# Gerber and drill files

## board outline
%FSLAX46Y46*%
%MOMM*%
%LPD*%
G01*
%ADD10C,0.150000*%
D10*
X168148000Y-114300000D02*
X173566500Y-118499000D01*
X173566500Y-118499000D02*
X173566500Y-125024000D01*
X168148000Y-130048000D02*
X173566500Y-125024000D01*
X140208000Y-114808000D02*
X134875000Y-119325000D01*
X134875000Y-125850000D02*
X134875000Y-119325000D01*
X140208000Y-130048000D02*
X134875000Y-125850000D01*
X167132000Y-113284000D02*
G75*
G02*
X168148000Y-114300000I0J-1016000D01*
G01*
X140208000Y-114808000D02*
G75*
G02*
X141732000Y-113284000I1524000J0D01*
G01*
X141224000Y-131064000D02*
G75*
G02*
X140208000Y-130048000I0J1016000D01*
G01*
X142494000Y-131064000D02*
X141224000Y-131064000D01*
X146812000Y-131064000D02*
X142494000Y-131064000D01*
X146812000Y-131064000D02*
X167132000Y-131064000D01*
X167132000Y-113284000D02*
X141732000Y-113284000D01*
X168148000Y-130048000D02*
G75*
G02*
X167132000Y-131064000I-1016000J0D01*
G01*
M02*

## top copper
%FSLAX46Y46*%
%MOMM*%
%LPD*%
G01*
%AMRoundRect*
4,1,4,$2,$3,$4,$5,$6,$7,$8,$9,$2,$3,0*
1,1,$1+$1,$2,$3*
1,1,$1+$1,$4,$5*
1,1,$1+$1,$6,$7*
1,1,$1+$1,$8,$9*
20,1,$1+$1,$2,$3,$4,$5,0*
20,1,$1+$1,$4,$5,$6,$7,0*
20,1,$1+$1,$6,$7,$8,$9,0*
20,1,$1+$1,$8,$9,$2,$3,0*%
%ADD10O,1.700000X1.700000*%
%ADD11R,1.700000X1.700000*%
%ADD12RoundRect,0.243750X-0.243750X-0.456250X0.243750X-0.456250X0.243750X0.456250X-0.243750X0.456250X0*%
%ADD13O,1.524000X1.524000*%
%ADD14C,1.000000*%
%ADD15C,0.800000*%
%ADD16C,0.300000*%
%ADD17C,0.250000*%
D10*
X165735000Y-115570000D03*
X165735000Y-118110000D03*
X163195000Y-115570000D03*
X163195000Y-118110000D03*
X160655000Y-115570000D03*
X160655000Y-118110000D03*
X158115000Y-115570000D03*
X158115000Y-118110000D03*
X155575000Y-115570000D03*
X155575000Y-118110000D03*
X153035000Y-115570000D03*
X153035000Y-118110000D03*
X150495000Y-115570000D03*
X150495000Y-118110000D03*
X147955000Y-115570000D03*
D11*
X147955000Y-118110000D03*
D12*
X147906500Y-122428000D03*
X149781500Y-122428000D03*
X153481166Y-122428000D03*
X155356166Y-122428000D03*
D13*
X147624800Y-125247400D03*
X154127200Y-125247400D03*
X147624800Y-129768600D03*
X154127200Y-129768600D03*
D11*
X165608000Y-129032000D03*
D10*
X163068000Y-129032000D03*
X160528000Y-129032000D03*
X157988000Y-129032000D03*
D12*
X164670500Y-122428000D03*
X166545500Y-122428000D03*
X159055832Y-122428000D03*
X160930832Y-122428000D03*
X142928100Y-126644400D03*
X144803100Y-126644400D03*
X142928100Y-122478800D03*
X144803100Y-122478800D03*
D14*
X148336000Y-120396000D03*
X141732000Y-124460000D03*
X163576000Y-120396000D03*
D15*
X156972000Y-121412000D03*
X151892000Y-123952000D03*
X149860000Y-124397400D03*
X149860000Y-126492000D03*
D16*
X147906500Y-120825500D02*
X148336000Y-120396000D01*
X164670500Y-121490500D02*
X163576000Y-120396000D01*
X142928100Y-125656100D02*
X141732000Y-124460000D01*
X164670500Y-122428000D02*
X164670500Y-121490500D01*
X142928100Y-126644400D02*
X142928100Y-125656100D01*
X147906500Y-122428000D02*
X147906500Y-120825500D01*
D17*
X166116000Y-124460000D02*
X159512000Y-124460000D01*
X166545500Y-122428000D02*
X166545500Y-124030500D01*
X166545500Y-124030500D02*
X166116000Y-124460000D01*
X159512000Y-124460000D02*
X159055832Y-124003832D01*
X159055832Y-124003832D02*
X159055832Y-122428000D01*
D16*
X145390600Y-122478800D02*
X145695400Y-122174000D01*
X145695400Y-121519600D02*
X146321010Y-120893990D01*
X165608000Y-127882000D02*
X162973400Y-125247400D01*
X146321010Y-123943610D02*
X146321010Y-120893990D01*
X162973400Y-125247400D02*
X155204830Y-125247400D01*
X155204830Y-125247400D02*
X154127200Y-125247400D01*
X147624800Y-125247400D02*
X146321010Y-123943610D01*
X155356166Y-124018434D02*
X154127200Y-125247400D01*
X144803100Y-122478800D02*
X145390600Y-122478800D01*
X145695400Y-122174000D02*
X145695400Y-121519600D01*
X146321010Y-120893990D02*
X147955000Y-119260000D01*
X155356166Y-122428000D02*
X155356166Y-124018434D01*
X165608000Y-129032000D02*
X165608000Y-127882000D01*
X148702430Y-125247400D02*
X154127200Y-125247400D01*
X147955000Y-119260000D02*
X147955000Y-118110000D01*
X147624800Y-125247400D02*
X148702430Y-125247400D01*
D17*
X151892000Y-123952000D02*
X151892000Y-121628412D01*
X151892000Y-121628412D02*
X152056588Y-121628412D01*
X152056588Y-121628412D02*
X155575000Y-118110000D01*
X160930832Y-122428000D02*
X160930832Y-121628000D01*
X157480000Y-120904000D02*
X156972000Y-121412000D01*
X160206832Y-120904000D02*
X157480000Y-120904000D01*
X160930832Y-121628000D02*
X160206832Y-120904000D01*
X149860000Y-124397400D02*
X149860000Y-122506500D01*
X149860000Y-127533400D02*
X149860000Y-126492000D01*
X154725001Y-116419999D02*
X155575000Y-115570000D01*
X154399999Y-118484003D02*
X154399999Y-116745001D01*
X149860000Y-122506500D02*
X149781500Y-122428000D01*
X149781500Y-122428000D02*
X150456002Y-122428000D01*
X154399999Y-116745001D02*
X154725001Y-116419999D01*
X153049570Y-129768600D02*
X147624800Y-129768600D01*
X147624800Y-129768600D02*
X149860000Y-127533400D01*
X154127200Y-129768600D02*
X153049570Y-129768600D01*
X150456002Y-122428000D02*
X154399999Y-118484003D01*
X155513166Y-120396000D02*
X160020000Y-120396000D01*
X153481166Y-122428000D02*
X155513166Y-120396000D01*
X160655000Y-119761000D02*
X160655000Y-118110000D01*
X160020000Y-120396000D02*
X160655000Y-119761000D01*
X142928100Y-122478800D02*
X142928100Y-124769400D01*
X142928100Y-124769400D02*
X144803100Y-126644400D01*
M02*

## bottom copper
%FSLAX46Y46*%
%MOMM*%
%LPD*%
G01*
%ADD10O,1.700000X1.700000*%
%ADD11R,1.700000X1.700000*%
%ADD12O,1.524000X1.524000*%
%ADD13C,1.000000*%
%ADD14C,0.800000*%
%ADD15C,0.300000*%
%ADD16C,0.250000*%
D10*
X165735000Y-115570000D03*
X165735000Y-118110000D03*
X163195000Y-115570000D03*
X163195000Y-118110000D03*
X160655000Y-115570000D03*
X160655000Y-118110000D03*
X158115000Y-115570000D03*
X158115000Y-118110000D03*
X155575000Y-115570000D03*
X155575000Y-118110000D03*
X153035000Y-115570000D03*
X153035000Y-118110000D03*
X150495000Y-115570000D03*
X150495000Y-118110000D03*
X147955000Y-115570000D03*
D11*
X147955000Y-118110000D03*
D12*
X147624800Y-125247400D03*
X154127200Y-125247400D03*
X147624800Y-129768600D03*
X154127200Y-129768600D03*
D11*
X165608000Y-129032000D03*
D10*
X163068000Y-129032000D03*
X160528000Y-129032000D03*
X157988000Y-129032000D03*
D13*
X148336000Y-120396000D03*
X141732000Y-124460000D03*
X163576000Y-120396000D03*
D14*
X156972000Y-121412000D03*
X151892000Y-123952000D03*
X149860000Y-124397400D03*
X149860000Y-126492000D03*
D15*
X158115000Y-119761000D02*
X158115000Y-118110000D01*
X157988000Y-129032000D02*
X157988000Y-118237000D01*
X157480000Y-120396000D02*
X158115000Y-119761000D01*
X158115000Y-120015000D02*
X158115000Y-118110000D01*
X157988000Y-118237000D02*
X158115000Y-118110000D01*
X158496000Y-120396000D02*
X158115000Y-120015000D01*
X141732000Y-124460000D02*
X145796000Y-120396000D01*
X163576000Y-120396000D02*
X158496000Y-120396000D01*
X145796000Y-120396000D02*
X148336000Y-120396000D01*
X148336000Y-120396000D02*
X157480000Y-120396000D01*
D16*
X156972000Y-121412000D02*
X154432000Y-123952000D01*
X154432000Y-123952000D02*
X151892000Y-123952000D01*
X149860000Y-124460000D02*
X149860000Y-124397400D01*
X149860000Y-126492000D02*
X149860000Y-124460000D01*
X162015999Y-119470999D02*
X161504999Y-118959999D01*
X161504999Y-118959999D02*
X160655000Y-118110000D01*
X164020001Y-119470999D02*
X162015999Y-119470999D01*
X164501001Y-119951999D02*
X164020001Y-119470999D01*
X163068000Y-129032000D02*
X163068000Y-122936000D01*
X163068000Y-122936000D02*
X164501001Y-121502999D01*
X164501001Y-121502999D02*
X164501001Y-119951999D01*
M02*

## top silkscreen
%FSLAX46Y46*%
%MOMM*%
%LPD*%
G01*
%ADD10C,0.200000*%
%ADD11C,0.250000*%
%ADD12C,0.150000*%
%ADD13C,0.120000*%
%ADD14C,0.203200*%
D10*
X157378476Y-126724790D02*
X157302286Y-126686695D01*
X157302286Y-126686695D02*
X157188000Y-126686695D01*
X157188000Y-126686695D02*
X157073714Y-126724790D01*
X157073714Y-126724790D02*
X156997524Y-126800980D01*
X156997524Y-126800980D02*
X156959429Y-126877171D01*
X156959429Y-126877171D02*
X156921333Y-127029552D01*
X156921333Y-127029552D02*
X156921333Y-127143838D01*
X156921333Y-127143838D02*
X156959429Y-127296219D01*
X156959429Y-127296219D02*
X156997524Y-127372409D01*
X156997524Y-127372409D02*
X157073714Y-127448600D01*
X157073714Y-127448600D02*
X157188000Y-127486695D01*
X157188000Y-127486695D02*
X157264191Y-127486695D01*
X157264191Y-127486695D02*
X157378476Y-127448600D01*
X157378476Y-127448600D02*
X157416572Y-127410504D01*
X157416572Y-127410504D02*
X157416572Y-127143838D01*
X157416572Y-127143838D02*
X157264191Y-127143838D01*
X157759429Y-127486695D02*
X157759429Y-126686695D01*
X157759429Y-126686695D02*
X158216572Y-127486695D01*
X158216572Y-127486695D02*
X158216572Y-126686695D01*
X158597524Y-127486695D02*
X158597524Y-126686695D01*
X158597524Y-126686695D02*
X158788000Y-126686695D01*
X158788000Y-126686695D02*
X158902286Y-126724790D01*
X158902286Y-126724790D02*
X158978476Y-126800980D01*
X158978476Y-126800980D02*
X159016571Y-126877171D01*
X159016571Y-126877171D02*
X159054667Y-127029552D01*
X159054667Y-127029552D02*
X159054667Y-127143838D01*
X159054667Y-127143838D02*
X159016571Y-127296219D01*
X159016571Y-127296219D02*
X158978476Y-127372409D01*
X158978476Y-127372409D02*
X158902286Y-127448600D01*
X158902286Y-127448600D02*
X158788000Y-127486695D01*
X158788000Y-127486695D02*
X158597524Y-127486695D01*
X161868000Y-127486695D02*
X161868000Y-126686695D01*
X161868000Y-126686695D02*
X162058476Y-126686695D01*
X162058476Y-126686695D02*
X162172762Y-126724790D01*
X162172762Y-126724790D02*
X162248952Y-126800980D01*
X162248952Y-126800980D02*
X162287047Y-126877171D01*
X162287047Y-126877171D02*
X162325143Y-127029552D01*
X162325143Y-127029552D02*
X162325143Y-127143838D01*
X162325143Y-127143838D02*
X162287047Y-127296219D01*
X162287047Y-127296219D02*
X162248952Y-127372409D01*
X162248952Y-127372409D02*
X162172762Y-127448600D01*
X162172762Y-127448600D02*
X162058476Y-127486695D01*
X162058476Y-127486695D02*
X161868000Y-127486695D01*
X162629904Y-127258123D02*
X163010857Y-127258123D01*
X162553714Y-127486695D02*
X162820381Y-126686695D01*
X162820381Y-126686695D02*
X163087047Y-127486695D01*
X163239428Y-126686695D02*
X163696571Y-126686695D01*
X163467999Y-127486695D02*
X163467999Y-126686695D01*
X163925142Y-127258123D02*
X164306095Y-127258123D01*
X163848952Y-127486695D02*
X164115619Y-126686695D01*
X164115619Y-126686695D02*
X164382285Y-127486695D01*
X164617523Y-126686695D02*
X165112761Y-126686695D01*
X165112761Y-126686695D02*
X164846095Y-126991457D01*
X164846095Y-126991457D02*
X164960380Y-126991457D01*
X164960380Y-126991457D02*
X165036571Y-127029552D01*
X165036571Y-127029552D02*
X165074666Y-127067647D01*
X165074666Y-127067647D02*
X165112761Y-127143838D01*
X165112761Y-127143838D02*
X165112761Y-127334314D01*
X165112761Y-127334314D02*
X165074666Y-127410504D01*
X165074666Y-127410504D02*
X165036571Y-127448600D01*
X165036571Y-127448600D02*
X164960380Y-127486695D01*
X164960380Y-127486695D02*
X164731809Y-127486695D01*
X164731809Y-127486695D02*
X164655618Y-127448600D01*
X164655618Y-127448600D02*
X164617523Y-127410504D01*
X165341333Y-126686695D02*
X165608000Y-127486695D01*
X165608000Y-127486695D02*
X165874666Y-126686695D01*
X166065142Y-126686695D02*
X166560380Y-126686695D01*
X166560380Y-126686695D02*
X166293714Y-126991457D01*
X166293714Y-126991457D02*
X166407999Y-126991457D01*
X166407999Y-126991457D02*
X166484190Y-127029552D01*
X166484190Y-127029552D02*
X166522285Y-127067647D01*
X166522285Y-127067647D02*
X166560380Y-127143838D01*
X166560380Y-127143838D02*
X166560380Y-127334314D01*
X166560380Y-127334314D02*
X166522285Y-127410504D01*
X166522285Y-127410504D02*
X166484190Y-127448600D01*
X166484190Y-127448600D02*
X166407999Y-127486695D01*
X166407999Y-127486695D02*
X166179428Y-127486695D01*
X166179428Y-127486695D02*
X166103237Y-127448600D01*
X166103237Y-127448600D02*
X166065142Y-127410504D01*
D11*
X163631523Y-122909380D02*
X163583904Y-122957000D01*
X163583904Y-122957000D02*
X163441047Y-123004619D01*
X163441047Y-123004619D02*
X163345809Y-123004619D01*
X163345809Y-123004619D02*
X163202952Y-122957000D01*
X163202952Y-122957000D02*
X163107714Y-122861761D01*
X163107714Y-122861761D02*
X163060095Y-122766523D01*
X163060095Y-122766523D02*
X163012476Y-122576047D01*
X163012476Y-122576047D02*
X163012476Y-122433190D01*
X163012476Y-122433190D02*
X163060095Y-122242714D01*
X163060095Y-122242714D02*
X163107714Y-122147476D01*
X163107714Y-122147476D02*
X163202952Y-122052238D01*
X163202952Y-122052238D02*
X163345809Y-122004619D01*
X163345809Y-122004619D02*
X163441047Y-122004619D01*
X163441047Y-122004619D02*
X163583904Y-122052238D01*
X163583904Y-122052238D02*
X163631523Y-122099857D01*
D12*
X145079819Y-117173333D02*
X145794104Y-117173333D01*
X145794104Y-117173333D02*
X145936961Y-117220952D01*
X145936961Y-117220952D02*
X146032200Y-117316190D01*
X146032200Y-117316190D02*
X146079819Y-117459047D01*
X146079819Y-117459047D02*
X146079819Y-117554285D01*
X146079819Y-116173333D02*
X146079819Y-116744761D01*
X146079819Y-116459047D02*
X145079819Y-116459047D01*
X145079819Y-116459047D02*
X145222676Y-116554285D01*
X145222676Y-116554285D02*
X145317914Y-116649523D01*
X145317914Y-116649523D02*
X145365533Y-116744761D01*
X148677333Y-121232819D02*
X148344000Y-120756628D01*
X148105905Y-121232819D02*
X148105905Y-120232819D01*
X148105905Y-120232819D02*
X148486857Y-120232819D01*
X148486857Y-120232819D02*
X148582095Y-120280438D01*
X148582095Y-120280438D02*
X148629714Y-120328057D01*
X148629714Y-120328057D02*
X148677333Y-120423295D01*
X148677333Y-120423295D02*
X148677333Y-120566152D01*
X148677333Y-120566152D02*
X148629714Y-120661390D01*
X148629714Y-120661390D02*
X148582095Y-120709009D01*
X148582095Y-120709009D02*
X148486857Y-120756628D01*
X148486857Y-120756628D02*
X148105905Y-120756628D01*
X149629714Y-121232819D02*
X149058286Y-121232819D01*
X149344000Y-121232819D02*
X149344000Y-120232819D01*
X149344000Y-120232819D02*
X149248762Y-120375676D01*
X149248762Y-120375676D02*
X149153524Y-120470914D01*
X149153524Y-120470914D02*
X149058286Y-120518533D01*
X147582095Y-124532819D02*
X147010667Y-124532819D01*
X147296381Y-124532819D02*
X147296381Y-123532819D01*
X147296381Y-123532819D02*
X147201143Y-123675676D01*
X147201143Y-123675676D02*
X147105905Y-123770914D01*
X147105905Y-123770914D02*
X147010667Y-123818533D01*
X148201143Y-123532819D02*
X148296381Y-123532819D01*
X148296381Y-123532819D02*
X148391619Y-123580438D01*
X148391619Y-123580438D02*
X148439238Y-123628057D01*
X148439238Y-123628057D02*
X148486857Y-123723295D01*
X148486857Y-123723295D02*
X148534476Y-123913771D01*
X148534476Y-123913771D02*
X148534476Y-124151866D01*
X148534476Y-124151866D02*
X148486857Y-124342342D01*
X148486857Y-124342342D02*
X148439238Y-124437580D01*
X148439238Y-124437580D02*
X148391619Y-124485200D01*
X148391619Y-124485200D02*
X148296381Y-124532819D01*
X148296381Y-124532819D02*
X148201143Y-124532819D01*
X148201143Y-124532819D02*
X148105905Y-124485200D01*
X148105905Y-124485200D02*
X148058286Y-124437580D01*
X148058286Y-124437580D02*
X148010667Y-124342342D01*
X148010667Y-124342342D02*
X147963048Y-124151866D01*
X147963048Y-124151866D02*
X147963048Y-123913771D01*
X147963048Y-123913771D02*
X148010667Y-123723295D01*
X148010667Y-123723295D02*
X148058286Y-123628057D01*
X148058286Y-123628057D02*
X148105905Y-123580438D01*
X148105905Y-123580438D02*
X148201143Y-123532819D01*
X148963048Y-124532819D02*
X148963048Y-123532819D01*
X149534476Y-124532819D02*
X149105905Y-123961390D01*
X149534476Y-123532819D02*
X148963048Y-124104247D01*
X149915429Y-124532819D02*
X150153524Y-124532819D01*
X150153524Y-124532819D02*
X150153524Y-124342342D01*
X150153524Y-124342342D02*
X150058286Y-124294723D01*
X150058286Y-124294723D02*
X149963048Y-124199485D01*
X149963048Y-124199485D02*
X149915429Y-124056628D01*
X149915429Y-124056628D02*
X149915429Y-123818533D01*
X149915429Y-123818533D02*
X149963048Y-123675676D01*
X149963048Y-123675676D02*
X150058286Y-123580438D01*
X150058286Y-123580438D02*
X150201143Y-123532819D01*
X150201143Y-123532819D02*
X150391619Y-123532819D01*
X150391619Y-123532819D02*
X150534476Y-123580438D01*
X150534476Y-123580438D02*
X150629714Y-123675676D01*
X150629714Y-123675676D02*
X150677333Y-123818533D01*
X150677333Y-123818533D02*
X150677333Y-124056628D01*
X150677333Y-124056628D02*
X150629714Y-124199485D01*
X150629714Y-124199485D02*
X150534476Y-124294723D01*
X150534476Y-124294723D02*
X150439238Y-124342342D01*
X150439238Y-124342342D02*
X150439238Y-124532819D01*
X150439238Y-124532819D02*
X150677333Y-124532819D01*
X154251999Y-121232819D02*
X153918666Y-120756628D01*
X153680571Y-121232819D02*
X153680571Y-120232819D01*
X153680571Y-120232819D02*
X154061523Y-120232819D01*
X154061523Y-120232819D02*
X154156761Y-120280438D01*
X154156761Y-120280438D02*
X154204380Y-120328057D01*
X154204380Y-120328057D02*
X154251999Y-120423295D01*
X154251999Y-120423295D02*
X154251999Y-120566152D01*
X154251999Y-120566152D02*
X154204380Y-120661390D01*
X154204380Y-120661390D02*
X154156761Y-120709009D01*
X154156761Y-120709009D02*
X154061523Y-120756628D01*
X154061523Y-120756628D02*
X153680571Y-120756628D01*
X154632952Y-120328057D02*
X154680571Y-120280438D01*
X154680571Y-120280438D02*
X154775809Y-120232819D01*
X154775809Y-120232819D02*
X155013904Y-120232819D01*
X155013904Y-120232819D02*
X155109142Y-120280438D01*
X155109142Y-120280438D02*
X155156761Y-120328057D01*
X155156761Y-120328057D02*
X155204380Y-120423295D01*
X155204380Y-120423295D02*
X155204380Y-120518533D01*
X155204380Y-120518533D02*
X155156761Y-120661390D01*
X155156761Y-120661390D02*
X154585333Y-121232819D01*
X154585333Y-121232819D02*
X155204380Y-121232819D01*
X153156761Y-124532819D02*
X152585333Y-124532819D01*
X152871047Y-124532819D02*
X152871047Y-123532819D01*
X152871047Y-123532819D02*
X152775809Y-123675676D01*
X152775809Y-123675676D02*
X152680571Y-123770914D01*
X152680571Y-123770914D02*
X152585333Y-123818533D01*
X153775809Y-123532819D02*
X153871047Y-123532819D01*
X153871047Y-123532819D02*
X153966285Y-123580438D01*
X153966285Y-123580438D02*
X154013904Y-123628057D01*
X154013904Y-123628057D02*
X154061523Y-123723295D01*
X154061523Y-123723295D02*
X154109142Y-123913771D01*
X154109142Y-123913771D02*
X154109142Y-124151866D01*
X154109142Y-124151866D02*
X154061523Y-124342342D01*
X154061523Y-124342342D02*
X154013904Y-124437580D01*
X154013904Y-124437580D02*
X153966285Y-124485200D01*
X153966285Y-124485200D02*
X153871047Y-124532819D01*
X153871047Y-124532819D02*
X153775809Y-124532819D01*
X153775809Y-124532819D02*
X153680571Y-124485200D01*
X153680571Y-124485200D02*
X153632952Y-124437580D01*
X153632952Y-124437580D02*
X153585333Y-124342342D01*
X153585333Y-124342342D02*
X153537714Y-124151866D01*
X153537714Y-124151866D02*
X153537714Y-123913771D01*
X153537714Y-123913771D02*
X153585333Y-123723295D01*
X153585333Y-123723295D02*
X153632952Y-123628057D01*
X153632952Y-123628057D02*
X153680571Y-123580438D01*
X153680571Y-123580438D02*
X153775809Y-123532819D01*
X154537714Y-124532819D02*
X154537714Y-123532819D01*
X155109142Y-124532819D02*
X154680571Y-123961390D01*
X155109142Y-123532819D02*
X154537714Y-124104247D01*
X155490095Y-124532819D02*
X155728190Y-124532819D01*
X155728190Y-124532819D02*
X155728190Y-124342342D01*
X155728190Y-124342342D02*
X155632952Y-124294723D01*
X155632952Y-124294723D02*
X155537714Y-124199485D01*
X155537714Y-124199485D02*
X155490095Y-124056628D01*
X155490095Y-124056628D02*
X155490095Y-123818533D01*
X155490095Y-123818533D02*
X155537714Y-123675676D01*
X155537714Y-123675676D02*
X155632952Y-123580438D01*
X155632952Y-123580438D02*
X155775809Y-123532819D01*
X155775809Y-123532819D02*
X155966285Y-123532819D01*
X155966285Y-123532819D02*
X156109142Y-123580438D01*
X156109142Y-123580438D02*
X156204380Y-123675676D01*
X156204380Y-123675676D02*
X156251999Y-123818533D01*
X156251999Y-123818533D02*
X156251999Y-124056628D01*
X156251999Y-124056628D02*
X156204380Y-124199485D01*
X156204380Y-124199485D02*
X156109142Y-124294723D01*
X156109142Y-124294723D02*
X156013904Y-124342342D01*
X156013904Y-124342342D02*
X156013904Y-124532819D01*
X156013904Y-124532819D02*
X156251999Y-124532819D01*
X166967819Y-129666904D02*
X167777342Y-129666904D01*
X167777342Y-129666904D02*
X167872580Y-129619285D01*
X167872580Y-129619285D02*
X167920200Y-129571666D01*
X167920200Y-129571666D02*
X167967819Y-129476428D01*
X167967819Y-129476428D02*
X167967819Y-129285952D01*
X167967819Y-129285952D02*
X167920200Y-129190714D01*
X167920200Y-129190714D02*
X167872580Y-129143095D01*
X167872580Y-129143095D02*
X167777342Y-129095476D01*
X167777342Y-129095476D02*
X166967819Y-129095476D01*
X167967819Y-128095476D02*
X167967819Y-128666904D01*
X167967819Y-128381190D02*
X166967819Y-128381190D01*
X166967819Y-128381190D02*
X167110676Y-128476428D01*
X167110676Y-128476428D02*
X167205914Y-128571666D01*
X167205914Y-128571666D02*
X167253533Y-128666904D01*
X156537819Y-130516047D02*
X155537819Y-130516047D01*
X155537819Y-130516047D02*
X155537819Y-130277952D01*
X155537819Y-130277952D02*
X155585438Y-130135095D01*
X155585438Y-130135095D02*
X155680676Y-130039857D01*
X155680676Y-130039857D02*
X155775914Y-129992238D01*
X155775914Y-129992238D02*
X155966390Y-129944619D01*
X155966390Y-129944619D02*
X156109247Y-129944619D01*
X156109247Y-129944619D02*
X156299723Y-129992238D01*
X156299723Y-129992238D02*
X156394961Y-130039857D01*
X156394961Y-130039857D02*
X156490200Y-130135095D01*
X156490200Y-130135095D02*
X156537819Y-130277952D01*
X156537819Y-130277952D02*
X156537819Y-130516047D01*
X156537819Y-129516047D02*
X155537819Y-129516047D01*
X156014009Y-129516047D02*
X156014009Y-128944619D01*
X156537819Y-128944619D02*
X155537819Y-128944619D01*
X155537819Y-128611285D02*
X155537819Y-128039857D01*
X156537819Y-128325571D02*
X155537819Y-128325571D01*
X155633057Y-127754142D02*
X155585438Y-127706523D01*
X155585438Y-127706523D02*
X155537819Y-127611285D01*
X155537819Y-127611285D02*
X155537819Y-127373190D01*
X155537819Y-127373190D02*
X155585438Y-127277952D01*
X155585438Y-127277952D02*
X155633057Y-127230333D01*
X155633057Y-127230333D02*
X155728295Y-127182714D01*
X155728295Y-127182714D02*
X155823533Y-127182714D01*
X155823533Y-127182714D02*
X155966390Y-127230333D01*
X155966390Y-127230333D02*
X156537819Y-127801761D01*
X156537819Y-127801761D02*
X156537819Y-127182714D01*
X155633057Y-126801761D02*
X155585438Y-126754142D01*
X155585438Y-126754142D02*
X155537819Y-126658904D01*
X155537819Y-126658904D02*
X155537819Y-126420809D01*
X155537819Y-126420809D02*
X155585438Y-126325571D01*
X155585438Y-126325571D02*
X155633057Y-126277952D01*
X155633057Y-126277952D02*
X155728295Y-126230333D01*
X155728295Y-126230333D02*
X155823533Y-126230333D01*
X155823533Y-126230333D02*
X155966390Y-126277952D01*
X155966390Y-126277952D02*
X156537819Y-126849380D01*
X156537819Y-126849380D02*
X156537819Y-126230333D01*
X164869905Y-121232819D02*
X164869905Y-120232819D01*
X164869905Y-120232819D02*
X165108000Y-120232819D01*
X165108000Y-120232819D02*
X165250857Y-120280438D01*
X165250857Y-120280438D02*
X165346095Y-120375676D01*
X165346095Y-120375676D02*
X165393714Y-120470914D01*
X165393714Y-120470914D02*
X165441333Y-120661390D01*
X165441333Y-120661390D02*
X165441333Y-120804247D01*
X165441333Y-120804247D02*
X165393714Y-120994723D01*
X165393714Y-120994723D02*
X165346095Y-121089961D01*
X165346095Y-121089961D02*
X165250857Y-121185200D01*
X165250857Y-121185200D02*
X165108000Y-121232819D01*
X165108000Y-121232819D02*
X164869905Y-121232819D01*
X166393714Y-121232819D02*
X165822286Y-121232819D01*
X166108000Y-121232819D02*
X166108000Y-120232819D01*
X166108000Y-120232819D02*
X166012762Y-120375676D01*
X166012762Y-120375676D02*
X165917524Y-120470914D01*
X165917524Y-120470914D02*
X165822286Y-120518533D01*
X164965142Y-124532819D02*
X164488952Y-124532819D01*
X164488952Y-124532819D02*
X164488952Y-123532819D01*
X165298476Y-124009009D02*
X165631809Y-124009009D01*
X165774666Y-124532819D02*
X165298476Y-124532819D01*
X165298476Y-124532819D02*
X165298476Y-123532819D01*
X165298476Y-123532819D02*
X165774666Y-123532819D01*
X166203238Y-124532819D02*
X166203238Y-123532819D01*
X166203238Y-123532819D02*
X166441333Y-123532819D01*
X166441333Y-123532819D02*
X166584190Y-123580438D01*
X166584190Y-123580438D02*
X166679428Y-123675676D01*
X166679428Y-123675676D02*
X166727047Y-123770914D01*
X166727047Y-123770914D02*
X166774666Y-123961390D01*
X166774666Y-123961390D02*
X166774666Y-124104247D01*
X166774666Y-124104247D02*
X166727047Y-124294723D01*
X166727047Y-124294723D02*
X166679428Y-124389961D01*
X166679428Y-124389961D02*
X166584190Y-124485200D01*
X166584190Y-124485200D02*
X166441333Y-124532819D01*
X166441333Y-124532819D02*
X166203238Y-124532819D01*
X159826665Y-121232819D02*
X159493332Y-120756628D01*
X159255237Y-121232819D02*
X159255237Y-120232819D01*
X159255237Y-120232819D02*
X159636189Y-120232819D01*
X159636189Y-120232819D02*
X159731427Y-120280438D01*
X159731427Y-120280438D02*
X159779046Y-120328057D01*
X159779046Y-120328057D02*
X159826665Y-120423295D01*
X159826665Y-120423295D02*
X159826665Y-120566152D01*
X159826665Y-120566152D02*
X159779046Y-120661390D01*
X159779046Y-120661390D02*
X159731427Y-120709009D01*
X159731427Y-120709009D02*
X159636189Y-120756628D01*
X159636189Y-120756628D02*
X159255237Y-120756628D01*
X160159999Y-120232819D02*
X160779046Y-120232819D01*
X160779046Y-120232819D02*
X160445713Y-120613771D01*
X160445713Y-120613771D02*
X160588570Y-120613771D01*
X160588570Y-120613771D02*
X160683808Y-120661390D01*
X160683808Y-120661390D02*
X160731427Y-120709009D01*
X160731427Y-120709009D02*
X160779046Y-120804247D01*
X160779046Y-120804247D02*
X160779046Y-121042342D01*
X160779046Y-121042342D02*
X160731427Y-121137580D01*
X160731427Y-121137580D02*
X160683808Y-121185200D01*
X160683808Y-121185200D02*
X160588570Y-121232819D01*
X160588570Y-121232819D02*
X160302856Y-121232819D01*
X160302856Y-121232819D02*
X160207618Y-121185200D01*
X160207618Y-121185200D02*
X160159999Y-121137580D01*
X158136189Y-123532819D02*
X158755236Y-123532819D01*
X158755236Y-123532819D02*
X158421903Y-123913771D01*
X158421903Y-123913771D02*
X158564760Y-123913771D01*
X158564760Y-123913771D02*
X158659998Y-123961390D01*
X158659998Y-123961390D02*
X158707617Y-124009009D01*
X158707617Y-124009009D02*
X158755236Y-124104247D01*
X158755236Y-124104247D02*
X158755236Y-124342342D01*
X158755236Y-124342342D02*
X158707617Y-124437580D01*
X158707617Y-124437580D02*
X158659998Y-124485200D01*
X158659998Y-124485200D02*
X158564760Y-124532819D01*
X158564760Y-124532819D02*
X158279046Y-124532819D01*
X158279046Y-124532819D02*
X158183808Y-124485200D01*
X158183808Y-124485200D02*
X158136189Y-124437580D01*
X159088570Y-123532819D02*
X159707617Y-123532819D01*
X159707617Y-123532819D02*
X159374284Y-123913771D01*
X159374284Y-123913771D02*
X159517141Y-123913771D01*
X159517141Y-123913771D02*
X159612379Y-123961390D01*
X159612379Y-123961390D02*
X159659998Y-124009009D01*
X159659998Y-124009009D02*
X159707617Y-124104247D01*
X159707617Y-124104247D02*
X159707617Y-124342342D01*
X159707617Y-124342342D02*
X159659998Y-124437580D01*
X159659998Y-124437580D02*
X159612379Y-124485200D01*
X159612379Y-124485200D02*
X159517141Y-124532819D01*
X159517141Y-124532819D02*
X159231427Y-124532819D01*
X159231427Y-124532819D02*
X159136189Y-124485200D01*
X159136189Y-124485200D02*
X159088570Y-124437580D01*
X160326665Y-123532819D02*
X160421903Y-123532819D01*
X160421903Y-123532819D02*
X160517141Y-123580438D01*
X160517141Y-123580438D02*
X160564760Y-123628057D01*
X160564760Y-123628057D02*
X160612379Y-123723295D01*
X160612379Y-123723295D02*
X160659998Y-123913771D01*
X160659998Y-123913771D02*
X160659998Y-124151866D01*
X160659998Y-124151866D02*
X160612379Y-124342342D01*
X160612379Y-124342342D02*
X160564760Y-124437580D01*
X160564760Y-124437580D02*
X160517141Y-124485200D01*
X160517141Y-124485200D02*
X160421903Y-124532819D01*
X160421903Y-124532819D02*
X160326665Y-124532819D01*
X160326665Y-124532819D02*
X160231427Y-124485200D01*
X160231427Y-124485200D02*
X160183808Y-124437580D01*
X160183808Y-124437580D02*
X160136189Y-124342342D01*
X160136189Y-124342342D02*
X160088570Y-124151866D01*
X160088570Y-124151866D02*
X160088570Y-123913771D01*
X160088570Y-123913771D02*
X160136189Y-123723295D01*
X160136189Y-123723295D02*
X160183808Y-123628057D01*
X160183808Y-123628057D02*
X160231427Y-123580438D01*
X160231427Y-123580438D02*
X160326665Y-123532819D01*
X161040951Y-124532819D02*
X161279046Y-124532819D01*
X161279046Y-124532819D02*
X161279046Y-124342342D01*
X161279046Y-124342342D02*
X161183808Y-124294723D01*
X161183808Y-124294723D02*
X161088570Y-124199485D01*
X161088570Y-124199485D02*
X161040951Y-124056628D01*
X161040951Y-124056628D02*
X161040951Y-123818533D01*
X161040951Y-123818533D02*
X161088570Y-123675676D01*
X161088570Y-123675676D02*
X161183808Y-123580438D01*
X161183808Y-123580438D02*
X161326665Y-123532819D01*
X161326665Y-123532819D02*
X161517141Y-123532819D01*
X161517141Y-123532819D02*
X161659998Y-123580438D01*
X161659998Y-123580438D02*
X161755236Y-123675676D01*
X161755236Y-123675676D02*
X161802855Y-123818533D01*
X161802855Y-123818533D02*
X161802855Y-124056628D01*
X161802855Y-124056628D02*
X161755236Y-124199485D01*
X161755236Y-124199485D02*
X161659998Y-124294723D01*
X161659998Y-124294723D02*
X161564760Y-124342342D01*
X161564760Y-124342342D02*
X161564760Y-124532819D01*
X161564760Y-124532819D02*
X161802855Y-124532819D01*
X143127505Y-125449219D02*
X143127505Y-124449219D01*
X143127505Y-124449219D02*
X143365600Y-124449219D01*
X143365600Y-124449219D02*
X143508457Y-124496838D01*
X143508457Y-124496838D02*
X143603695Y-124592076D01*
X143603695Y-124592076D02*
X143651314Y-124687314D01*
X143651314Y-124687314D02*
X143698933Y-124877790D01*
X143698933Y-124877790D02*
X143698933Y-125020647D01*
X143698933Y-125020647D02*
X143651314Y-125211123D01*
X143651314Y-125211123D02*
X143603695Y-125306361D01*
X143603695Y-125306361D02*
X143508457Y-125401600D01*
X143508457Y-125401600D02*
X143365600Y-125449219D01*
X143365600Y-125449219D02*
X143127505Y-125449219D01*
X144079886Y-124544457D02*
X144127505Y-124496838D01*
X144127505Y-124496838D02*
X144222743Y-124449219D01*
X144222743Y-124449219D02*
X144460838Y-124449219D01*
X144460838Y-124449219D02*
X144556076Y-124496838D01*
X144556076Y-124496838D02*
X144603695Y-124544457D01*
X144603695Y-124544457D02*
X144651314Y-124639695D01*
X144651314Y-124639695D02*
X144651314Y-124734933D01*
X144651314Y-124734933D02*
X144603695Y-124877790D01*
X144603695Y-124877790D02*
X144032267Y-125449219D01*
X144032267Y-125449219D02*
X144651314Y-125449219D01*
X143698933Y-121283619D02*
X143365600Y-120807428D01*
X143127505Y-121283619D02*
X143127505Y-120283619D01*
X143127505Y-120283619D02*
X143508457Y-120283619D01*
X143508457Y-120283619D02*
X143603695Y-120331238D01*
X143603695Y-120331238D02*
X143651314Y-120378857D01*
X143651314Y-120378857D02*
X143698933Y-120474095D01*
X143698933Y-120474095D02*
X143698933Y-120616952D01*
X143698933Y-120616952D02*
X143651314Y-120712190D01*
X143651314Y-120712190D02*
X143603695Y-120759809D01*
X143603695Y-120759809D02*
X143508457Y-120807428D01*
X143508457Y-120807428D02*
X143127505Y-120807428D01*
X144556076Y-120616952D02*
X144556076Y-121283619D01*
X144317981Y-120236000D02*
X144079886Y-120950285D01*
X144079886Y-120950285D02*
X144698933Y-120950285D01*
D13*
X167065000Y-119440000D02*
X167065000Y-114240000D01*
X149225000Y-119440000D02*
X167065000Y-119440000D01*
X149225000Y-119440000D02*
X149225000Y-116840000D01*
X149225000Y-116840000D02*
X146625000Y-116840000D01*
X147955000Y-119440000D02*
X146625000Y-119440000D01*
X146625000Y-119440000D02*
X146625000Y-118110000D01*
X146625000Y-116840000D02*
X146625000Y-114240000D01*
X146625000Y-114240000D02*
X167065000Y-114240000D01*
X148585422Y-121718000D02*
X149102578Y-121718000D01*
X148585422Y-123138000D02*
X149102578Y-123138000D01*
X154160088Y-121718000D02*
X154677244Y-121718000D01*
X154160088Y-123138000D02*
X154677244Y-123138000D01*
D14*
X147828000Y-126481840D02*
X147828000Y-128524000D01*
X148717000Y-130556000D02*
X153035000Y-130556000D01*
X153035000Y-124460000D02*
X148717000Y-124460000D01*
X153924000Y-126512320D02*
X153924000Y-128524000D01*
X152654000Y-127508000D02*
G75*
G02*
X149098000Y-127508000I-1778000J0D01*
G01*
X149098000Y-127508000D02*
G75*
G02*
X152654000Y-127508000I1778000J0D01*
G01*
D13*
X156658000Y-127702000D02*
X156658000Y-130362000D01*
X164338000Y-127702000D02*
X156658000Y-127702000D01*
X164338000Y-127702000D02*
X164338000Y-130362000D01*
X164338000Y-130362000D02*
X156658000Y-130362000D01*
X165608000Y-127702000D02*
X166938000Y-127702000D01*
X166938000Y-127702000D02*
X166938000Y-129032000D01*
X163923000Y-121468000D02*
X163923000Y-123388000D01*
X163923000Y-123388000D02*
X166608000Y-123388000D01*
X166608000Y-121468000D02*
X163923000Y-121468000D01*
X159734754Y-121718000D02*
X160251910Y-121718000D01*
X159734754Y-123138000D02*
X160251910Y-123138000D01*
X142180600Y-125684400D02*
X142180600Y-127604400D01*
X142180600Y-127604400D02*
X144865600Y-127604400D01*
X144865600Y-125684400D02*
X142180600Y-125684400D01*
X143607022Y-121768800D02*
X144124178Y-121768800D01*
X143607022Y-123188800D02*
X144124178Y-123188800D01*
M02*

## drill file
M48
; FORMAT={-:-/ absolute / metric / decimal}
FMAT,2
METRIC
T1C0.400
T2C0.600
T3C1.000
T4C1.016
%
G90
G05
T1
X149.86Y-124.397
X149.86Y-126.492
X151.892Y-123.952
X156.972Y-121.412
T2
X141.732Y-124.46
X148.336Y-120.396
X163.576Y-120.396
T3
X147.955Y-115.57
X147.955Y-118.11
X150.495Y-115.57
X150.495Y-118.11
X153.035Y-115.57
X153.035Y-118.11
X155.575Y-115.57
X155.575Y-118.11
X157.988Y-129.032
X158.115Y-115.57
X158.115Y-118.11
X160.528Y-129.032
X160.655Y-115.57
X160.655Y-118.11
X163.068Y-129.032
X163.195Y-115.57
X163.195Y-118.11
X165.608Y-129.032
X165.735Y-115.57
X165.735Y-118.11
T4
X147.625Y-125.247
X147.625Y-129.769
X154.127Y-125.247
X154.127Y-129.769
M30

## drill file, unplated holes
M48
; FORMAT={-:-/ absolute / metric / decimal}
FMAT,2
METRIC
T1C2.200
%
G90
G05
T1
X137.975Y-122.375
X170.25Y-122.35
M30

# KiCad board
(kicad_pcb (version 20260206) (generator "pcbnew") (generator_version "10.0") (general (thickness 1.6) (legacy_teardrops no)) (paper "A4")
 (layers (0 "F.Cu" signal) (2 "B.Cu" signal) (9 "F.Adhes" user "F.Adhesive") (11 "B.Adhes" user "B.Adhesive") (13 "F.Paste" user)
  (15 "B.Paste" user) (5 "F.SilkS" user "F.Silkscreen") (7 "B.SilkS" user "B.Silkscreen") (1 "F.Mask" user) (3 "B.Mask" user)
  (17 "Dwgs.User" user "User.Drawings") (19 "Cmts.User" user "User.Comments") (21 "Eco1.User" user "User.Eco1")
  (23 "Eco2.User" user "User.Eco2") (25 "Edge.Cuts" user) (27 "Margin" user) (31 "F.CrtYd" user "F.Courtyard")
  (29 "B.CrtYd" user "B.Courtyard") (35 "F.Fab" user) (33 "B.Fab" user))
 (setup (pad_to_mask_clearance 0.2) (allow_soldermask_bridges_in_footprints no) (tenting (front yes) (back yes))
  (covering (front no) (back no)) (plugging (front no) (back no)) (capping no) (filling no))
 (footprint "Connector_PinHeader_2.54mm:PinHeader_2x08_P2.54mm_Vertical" (layer "F.Cu") (at 147.955 118.11 90)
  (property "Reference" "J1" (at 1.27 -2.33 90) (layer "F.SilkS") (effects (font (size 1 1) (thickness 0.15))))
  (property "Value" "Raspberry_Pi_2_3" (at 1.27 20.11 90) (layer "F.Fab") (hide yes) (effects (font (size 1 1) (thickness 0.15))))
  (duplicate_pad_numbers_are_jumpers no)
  (fp_line (start 3.87 -1.33) (end 3.87 19.11) (stroke (width 0.12) (type solid)) (layer "F.SilkS"))
  (fp_line (start 1.27 -1.33) (end 3.87 -1.33) (stroke (width 0.12) (type solid)) (layer "F.SilkS"))
  (fp_line (start -1.33 -1.33) (end 0 -1.33) (stroke (width 0.12) (type solid)) (layer "F.SilkS"))
  (fp_line (start -1.33 0) (end -1.33 -1.33) (stroke (width 0.12) (type solid)) (layer "F.SilkS"))
  (fp_line (start 1.27 1.27) (end 1.27 -1.33) (stroke (width 0.12) (type solid)) (layer "F.SilkS"))
  (fp_line (start -1.33 1.27) (end 1.27 1.27) (stroke (width 0.12) (type solid)) (layer "F.SilkS"))
  (fp_line (start -1.33 1.27) (end -1.33 19.11) (stroke (width 0.12) (type solid)) (layer "F.SilkS"))
  (fp_line (start -1.33 19.11) (end 3.87 19.11) (stroke (width 0.12) (type solid)) (layer "F.SilkS"))
  (pad "1" thru_hole rect (at 0 0 90) (size 1.7 1.7) (drill 1) (layers "*.Cu" "*.Mask") (remove_unused_layers no) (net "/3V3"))
  (pad "2" thru_hole oval (at 2.54 0 90) (size 1.7 1.7) (drill 1) (layers "*.Cu" "*.Mask") (remove_unused_layers no) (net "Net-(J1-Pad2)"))
  (pad "3" thru_hole oval (at 0 2.54 90) (size 1.7 1.7) (drill 1) (layers "*.Cu" "*.Mask") (remove_unused_layers no) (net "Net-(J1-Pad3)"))
  (pad "4" thru_hole oval (at 2.54 2.54 90) (size 1.7 1.7) (drill 1) (layers "*.Cu" "*.Mask") (remove_unused_layers no)
   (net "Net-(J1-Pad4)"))
  (pad "5" thru_hole oval (at 0 5.08 90) (size 1.7 1.7) (drill 1) (layers "*.Cu" "*.Mask") (remove_unused_layers no) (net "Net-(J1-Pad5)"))
  (pad "6" thru_hole oval (at 2.54 5.08 90) (size 1.7 1.7) (drill 1) (layers "*.Cu" "*.Mask") (remove_unused_layers no) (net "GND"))
  (pad "7" thru_hole oval (at 0 7.62 90) (size 1.7 1.7) (drill 1) (layers "*.Cu" "*.Mask") (remove_unused_layers no) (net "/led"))
  (pad "8" thru_hole oval (at 2.54 7.62 90) (size 1.7 1.7) (drill 1) (layers "*.Cu" "*.Mask") (remove_unused_layers no)
   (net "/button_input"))
  (pad "9" thru_hole oval (at 0 10.16 90) (size 1.7 1.7) (drill 1) (layers "*.Cu" "*.Mask") (remove_unused_layers no) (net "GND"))
  (pad "10" thru_hole oval (at 2.54 10.16 90) (size 1.7 1.7) (drill 1) (layers "*.Cu" "*.Mask") (remove_unused_layers no)
   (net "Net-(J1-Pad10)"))
  (pad "11" thru_hole oval (at 0 12.7 90) (size 1.7 1.7) (drill 1) (layers "*.Cu" "*.Mask") (remove_unused_layers no) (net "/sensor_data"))
  (pad "12" thru_hole oval (at 2.54 12.7 90) (size 1.7 1.7) (drill 1) (layers "*.Cu" "*.Mask") (remove_unused_layers no)
   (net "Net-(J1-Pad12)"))
  (pad "13" thru_hole oval (at 0 15.24 90) (size 1.7 1.7) (drill 1) (layers "*.Cu" "*.Mask") (remove_unused_layers no)
   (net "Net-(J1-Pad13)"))
  (pad "14" thru_hole oval (at 2.54 15.24 90) (size 1.7 1.7) (drill 1) (layers "*.Cu" "*.Mask") (remove_unused_layers no)
   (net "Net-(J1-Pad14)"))
  (pad "15" thru_hole oval (at 0 17.78 90) (size 1.7 1.7) (drill 1) (layers "*.Cu" "*.Mask") (remove_unused_layers no)
   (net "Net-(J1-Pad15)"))
  (pad "16" thru_hole oval (at 2.54 17.78 90) (size 1.7 1.7) (drill 1) (layers "*.Cu" "*.Mask") (remove_unused_layers no)
   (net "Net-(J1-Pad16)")))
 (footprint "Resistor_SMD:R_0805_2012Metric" (layer "F.Cu") (at 148.844 122.428)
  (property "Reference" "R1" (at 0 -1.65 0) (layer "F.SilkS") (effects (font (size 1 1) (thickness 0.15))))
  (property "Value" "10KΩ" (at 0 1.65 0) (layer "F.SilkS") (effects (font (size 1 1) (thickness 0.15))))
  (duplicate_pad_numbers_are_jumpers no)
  (fp_line (start -0.258578 -0.71) (end 0.258578 -0.71) (stroke (width 0.12) (type solid)) (layer "F.SilkS"))
  (fp_line (start -0.258578 0.71) (end 0.258578 0.71) (stroke (width 0.12) (type solid)) (layer "F.SilkS"))
  (pad "1" smd roundrect (at -0.9375 0) (size 0.975 1.4) (layers "F.Cu" "F.Mask" "F.Paste") (roundrect_rratio 0.25) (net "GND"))
  (pad "2" smd roundrect (at 0.9375 0) (size 0.975 1.4) (layers "F.Cu" "F.Mask" "F.Paste") (roundrect_rratio 0.25) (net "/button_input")))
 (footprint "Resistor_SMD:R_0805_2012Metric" (layer "F.Cu") (at 154.418666 122.428)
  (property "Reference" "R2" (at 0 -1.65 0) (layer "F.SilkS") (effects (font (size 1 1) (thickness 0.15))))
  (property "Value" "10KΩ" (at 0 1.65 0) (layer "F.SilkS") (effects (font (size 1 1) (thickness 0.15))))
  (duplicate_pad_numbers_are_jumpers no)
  (fp_line (start -0.258578 -0.71) (end 0.258578 -0.71) (stroke (width 0.12) (type solid)) (layer "F.SilkS"))
  (fp_line (start -0.258578 0.71) (end 0.258578 0.71) (stroke (width 0.12) (type solid)) (layer "F.SilkS"))
  (pad "1" smd roundrect (at -0.9375 0) (size 0.975 1.4) (layers "F.Cu" "F.Mask" "F.Paste") (roundrect_rratio 0.25) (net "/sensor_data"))
  (pad "2" smd roundrect (at 0.9375 0) (size 0.975 1.4) (layers "F.Cu" "F.Mask" "F.Paste") (roundrect_rratio 0.25) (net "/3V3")))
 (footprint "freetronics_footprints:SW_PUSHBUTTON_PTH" (layer "F.Cu") (at 150.876 127.508)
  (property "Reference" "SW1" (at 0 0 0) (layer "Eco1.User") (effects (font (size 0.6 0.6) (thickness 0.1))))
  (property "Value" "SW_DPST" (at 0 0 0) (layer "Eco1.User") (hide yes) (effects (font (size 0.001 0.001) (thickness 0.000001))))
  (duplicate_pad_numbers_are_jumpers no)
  (fp_line (start -3.048 -1.02616) (end -3.048 1.016) (stroke (width 0.2032) (type solid)) (layer "F.SilkS"))
  (fp_line (start -2.159 3.048) (end 2.159 3.048) (stroke (width 0.2032) (type solid)) (layer "F.SilkS"))
  (fp_line (start 2.159 -3.048) (end -2.159 -3.048) (stroke (width 0.2032) (type solid)) (layer "F.SilkS"))
  (fp_line (start 3.048 -0.99568) (end 3.048 1.016) (stroke (width 0.2032) (type solid)) (layer "F.SilkS"))
  (fp_circle (center 0 0) (end 1.778 0) (stroke (width 0.2032) (type solid)) (fill no) (layer "F.SilkS"))
  (pad "1" thru_hole oval (at -3.2512 -2.2606) (size 1.524 1.524) (drill 1.016) (layers "*.Cu" "*.Mask") (remove_unused_layers no)
   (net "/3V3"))
  (pad "1" thru_hole oval (at 3.2512 -2.2606) (size 1.524 1.524) (drill 1.016) (layers "*.Cu" "*.Mask") (remove_unused_layers no)
   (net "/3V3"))
  (pad "2" thru_hole oval (at -3.2512 2.2606) (size 1.524 1.524) (drill 1.016) (layers "*.Cu" "*.Mask") (remove_unused_layers no)
   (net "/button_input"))
  (pad "2" thru_hole oval (at 3.2512 2.2606) (size 1.524 1.524) (drill 1.016) (layers "*.Cu" "*.Mask") (remove_unused_layers no)
   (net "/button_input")))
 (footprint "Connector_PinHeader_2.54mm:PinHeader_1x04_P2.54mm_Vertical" (layer "F.Cu") (at 165.608 129.032 -90)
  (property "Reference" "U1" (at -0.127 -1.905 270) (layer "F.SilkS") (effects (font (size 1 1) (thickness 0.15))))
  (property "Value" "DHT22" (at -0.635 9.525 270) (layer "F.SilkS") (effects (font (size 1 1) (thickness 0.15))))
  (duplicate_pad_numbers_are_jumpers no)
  (fp_line (start -1.33 8.95) (end 1.33 8.95) (stroke (width 0.12) (type solid)) (layer "F.SilkS"))
  (fp_line (start -1.33 1.27) (end -1.33 8.95) (stroke (width 0.12) (type solid)) (layer "F.SilkS"))
  (fp_line (start -1.33 1.27) (end 1.33 1.27) (stroke (width 0.12) (type solid)) (layer "F.SilkS"))
  (fp_line (start 1.33 1.27) (end 1.33 8.95) (stroke (width 0.12) (type solid)) (layer "F.SilkS"))
  (fp_line (start -1.33 0) (end -1.33 -1.33) (stroke (width 0.12) (type solid)) (layer "F.SilkS"))
  (fp_line (start -1.33 -1.33) (end 0 -1.33) (stroke (width 0.12) (type solid)) (layer "F.SilkS"))
  (pad "1" thru_hole rect (at 0 0 270) (size 1.7 1.7) (drill 1) (layers "*.Cu" "*.Mask") (remove_unused_layers no) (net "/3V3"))
  (pad "2" thru_hole oval (at 0 2.54 270) (size 1.7 1.7) (drill 1) (layers "*.Cu" "*.Mask") (remove_unused_layers no) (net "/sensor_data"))
  (pad "3" thru_hole oval (at 0 5.08 270) (size 1.7 1.7) (drill 1) (layers "*.Cu" "*.Mask") (remove_unused_layers no))
  (pad "4" thru_hole oval (at 0 7.62 270) (size 1.7 1.7) (drill 1) (layers "*.Cu" "*.Mask") (remove_unused_layers no) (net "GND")))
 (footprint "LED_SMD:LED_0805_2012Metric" (layer "F.Cu") (at 165.608 122.428)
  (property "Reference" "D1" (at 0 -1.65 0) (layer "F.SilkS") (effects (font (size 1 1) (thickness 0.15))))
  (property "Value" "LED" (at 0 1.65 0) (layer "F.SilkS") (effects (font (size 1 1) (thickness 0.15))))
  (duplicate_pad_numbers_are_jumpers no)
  (fp_line (start -1.685 -0.96) (end -1.685 0.96) (stroke (width 0.12) (type solid)) (layer "F.SilkS"))
  (fp_line (start -1.685 0.96) (end 1 0.96) (stroke (width 0.12) (type solid)) (layer "F.SilkS"))
  (fp_line (start 1 -0.96) (end -1.685 -0.96) (stroke (width 0.12) (type solid)) (layer "F.SilkS"))
  (pad "1" smd roundrect (at -0.9375 0) (size 0.975 1.4) (layers "F.Cu" "F.Mask" "F.Paste") (roundrect_rratio 0.25) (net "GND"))
  (pad "2" smd roundrect (at 0.9375 0) (size 0.975 1.4) (layers "F.Cu" "F.Mask" "F.Paste") (roundrect_rratio 0.25) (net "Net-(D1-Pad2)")))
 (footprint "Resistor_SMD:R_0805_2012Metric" (layer "F.Cu") (at 159.993332 122.428)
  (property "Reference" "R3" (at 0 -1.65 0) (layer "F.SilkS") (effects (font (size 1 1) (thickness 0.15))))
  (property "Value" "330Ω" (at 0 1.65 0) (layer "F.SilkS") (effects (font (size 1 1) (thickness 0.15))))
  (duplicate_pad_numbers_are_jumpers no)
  (fp_line (start -0.258578 -0.71) (end 0.258578 -0.71) (stroke (width 0.12) (type solid)) (layer "F.SilkS"))
  (fp_line (start -0.258578 0.71) (end 0.258578 0.71) (stroke (width 0.12) (type solid)) (layer "F.SilkS"))
  (pad "1" smd roundrect (at -0.9375 0) (size 0.975 1.4) (layers "F.Cu" "F.Mask" "F.Paste") (roundrect_rratio 0.25) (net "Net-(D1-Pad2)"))
  (pad "2" smd roundrect (at 0.9375 0) (size 0.975 1.4) (layers "F.Cu" "F.Mask" "F.Paste") (roundrect_rratio 0.25) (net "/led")))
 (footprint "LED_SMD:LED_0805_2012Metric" (layer "F.Cu") (at 143.8656 126.6444)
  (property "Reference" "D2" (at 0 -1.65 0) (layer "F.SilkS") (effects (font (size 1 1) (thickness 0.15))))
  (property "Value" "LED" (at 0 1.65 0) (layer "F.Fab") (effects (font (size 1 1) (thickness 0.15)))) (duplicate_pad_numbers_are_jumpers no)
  (fp_line (start -1.685 -0.96) (end -1.685 0.96) (stroke (width 0.12) (type solid)) (layer "F.SilkS"))
  (fp_line (start -1.685 0.96) (end 1 0.96) (stroke (width 0.12) (type solid)) (layer "F.SilkS"))
  (fp_line (start 1 -0.96) (end -1.685 -0.96) (stroke (width 0.12) (type solid)) (layer "F.SilkS"))
  (pad "1" smd roundrect (at -0.9375 0) (size 0.975 1.4) (layers "F.Cu" "F.Mask" "F.Paste") (roundrect_rratio 0.25) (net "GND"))
  (pad "2" smd roundrect (at 0.9375 0) (size 0.975 1.4) (layers "F.Cu" "F.Mask" "F.Paste") (roundrect_rratio 0.25) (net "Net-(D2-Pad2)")))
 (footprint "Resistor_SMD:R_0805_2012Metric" (layer "F.Cu") (at 143.8656 122.4788)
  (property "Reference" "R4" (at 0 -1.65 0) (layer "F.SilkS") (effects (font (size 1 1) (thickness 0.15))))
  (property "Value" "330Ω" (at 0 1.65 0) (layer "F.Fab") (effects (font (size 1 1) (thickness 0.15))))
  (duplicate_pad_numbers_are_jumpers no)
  (fp_line (start -0.258578 -0.71) (end 0.258578 -0.71) (stroke (width 0.12) (type solid)) (layer "F.SilkS"))
  (fp_line (start -0.258578 0.71) (end 0.258578 0.71) (stroke (width 0.12) (type solid)) (layer "F.SilkS"))
  (pad "1" smd roundrect (at -0.9375 0) (size 0.975 1.4) (layers "F.Cu" "F.Mask" "F.Paste") (roundrect_rratio 0.25) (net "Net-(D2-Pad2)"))
  (pad "2" smd roundrect (at 0.9375 0) (size 0.975 1.4) (layers "F.Cu" "F.Mask" "F.Paste") (roundrect_rratio 0.25) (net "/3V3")))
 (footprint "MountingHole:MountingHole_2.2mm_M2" (layer "F.Cu") (at 170.25 122.35)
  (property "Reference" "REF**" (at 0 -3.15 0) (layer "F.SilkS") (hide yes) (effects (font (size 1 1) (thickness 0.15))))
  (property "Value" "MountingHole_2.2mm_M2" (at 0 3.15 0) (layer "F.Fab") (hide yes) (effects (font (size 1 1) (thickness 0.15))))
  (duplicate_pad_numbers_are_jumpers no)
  (pad "" np_thru_hole circle (at 0 0) (size 2.2 2.2) (drill 2.2) (layers "*.Cu" "*.Mask")))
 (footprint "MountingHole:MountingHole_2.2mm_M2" (layer "F.Cu") (at 137.975 122.375)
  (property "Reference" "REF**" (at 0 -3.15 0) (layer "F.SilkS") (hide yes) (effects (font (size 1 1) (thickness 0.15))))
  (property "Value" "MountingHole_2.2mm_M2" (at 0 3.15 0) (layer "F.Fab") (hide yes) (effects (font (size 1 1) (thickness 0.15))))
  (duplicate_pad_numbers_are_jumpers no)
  (pad "" np_thru_hole circle (at 0 0) (size 2.2 2.2) (drill 2.2) (layers "*.Cu" "*.Mask")))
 (gr_line (start 134.875 125.85) (end 134.875 119.325) (stroke (width 0.15) (type solid)) (layer "Edge.Cuts"))
 (gr_line (start 140.208 114.808) (end 134.875 119.325) (stroke (width 0.15) (type solid)) (layer "Edge.Cuts"))
 (gr_arc (start 140.208 114.808) (mid 140.654369 113.730369) (end 141.732 113.284) (stroke (width 0.15) (type solid)) (layer "Edge.Cuts"))
 (gr_line (start 140.208 130.048) (end 134.875 125.85) (stroke (width 0.15) (type solid)) (layer "Edge.Cuts"))
 (gr_arc (start 141.224 131.064) (mid 140.50558 130.76642) (end 140.208 130.048) (stroke (width 0.15) (type solid)) (layer "Edge.Cuts"))
 (gr_line (start 142.494 131.064) (end 141.224 131.064) (stroke (width 0.15) (type solid)) (layer "Edge.Cuts"))
 (gr_line (start 146.812 131.064) (end 142.494 131.064) (stroke (width 0.15) (type solid)) (layer "Edge.Cuts"))
 (gr_line (start 146.812 131.064) (end 167.132 131.064) (stroke (width 0.15) (type solid)) (layer "Edge.Cuts"))
 (gr_line (start 167.132 113.284) (end 141.732 113.284) (stroke (width 0.15) (type solid)) (layer "Edge.Cuts"))
 (gr_arc (start 167.132 113.284) (mid 167.85042 113.58158) (end 168.148 114.3) (stroke (width 0.15) (type solid)) (layer "Edge.Cuts"))
 (gr_line (start 168.148 114.3) (end 173.5665 118.499) (stroke (width 0.15) (type solid)) (layer "Edge.Cuts"))
 (gr_arc (start 168.148 130.048) (mid 167.85042 130.76642) (end 167.132 131.064) (stroke (width 0.15) (type solid)) (layer "Edge.Cuts"))
 (gr_line (start 168.148 130.048) (end 173.5665 125.024) (stroke (width 0.15) (type solid)) (layer "Edge.Cuts"))
 (gr_line (start 173.5665 118.499) (end 173.5665 125.024) (stroke (width 0.15) (type solid)) (layer "Edge.Cuts"))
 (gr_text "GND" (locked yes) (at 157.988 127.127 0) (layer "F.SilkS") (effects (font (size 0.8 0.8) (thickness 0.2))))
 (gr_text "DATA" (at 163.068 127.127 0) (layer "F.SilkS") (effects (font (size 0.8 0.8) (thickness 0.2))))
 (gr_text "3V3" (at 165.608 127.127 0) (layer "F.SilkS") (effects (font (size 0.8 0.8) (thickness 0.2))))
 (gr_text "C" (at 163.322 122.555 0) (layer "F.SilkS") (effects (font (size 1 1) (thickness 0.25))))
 (segment (start 145.3906 122.4788) (end 145.6954 122.174) (width 0.3) (layer "F.Cu") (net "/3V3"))
 (segment (start 145.6954 121.5196) (end 146.32101 120.89399) (width 0.3) (layer "F.Cu") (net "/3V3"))
 (segment (start 165.608 127.882) (end 162.9734 125.2474) (width 0.3) (layer "F.Cu") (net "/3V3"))
 (segment (start 146.32101 123.94361) (end 146.32101 120.89399) (width 0.3) (layer "F.Cu") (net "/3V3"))
 (segment (start 162.9734 125.2474) (end 155.20483 125.2474) (width 0.3) (layer "F.Cu") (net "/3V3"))
 (segment (start 155.20483 125.2474) (end 154.1272 125.2474) (width 0.3) (layer "F.Cu") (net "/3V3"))
 (segment (start 147.6248 125.2474) (end 146.32101 123.94361) (width 0.3) (layer "F.Cu") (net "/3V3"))
 (segment (start 155.356166 124.018434) (end 154.1272 125.2474) (width 0.3) (layer "F.Cu") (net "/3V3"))
 (segment (start 144.8031 122.4788) (end 145.3906 122.4788) (width 0.3) (layer "F.Cu") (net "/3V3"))
 (segment (start 145.6954 122.174) (end 145.6954 121.5196) (width 0.3) (layer "F.Cu") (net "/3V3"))
 (segment (start 146.32101 120.89399) (end 147.955 119.26) (width 0.3) (layer "F.Cu") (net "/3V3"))
 (segment (start 155.356166 122.428) (end 155.356166 124.018434) (width 0.3) (layer "F.Cu") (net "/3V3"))
 (segment (start 165.608 129.032) (end 165.608 127.882) (width 0.3) (layer "F.Cu") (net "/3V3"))
 (segment (start 148.70243 125.2474) (end 154.1272 125.2474) (width 0.3) (layer "F.Cu") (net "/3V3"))
 (segment (start 147.955 119.26) (end 147.955 118.11) (width 0.3) (layer "F.Cu") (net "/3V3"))
 (segment (start 147.6248 125.2474) (end 148.70243 125.2474) (width 0.3) (layer "F.Cu") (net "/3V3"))
 (segment (start 147.9065 120.8255) (end 148.336 120.396) (width 0.3) (layer "F.Cu") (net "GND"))
 (segment (start 164.6705 121.4905) (end 163.576 120.396) (width 0.3) (layer "F.Cu") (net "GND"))
 (segment (start 142.9281 125.6561) (end 141.732 124.46) (width 0.3) (layer "F.Cu") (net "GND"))
 (segment (start 164.6705 122.428) (end 164.6705 121.4905) (width 0.3) (layer "F.Cu") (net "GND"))
 (segment (start 142.9281 126.6444) (end 142.9281 125.6561) (width 0.3) (layer "F.Cu") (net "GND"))
 (segment (start 147.9065 122.428) (end 147.9065 120.8255) (width 0.3) (layer "F.Cu") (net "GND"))
 (via (at 148.336 120.396) (size 1) (drill 0.6) (layers "F.Cu" "B.Cu") (capping no) (covering (front no) (back no))
  (plugging (front no) (back no)) (filling no) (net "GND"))
 (via (at 141.732 124.46) (size 1) (drill 0.6) (layers "F.Cu" "B.Cu") (capping no) (covering (front no) (back no))
  (plugging (front no) (back no)) (filling no) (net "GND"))
 (via (at 163.576 120.396) (size 1) (drill 0.6) (layers "F.Cu" "B.Cu") (capping no) (covering (front no) (back no))
  (plugging (front no) (back no)) (filling no) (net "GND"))
 (segment (start 158.115 119.761) (end 158.115 118.11) (width 0.3) (layer "B.Cu") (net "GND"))
 (segment (start 157.988 129.032) (end 157.988 118.237) (width 0.3) (layer "B.Cu") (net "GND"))
 (segment (start 157.48 120.396) (end 158.115 119.761) (width 0.3) (layer "B.Cu") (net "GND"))
 (segment (start 158.115 120.015) (end 158.115 118.11) (width 0.3) (layer "B.Cu") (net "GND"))
 (segment (start 157.988 118.237) (end 158.115 118.11) (width 0.3) (layer "B.Cu") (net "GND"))
 (segment (start 158.496 120.396) (end 158.115 120.015) (width 0.3) (layer "B.Cu") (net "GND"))
 (segment (start 141.732 124.46) (end 145.796 120.396) (width 0.3) (layer "B.Cu") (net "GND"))
 (segment (start 163.576 120.396) (end 158.496 120.396) (width 0.3) (layer "B.Cu") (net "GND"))
 (segment (start 145.796 120.396) (end 148.336 120.396) (width 0.3) (layer "B.Cu") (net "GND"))
 (segment (start 148.336 120.396) (end 157.48 120.396) (width 0.3) (layer "B.Cu") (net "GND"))
 (segment (start 151.892 123.952) (end 151.892 121.628412) (width 0.25) (layer "F.Cu") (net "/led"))
 (segment (start 151.892 121.628412) (end 152.056588 121.628412) (width 0.25) (layer "F.Cu") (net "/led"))
 (segment (start 152.056588 121.628412) (end 155.575 118.11) (width 0.25) (layer "F.Cu") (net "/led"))
 (segment (start 160.930832 122.428) (end 160.930832 121.628) (width 0.25) (layer "F.Cu") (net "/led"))
 (segment (start 157.48 120.904) (end 156.972 121.412) (width 0.25) (layer "F.Cu") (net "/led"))
 (segment (start 160.206832 120.904) (end 157.48 120.904) (width 0.25) (layer "F.Cu") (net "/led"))
 (segment (start 160.930832 121.628) (end 160.206832 120.904) (width 0.25) (layer "F.Cu") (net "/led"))
 (via (at 156.972 121.412) (size 0.8) (drill 0.4) (layers "F.Cu" "B.Cu") (capping no) (covering (front no) (back no))
  (plugging (front no) (back no)) (filling no) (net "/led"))
 (via (at 151.892 123.952) (size 0.8) (drill 0.4) (layers "F.Cu" "B.Cu") (capping no) (covering (front no) (back no))
  (plugging (front no) (back no)) (filling no) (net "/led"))
 (segment (start 156.972 121.412) (end 154.432 123.952) (width 0.25) (layer "B.Cu") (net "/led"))
 (segment (start 154.432 123.952) (end 151.892 123.952) (width 0.25) (layer "B.Cu") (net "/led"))
 (segment (start 149.86 124.3974) (end 149.86 122.5065) (width 0.25) (layer "F.Cu") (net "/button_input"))
 (segment (start 149.86 127.5334) (end 149.86 126.492) (width 0.25) (layer "F.Cu") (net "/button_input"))
 (segment (start 154.725001 116.419999) (end 155.575 115.57) (width 0.25) (layer "F.Cu") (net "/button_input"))
 (segment (start 154.399999 118.484003) (end 154.399999 116.745001) (width 0.25) (layer "F.Cu") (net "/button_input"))
 (segment (start 149.86 122.5065) (end 149.7815 122.428) (width 0.25) (layer "F.Cu") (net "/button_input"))
 (segment (start 149.7815 122.428) (end 150.456002 122.428) (width 0.25) (layer "F.Cu") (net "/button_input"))
 (segment (start 154.399999 116.745001) (end 154.725001 116.419999) (width 0.25) (layer "F.Cu") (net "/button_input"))
 (segment (start 153.04957 129.7686) (end 147.6248 129.7686) (width 0.25) (layer "F.Cu") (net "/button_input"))
 (segment (start 147.6248 129.7686) (end 149.86 127.5334) (width 0.25) (layer "F.Cu") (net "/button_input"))
 (segment (start 154.1272 129.7686) (end 153.04957 129.7686) (width 0.25) (layer "F.Cu") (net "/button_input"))
 (segment (start 150.456002 122.428) (end 154.399999 118.484003) (width 0.25) (layer "F.Cu") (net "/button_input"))
 (via (at 149.86 124.3974) (size 0.8) (drill 0.4) (layers "F.Cu" "B.Cu") (capping no) (covering (front no) (back no))
  (plugging (front no) (back no)) (filling no) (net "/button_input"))
 (via (at 149.86 126.492) (size 0.8) (drill 0.4) (layers "F.Cu" "B.Cu") (capping no) (covering (front no) (back no))
  (plugging (front no) (back no)) (filling no) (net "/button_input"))
 (segment (start 149.86 124.46) (end 149.86 124.3974) (width 0.25) (layer "B.Cu") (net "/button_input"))
 (segment (start 149.86 126.492) (end 149.86 124.46) (width 0.25) (layer "B.Cu") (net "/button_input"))
 (segment (start 155.513166 120.396) (end 160.02 120.396) (width 0.25) (layer "F.Cu") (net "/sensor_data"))
 (segment (start 153.481166 122.428) (end 155.513166 120.396) (width 0.25) (layer "F.Cu") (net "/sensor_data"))
 (segment (start 160.655 119.761) (end 160.655 118.11) (width 0.25) (layer "F.Cu") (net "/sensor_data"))
 (segment (start 160.02 120.396) (end 160.655 119.761) (width 0.25) (layer "F.Cu") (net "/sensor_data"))
 (segment (start 162.015999 119.470999) (end 161.504999 118.959999) (width 0.25) (layer "B.Cu") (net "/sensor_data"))
 (segment (start 161.504999 118.959999) (end 160.655 118.11) (width 0.25) (layer "B.Cu") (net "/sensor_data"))
 (segment (start 164.020001 119.470999) (end 162.015999 119.470999) (width 0.25) (layer "B.Cu") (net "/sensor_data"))
 (segment (start 164.501001 119.951999) (end 164.020001 119.470999) (width 0.25) (layer "B.Cu") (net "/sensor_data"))
 (segment (start 163.068 129.032) (end 163.068 122.936) (width 0.25) (layer "B.Cu") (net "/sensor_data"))
 (segment (start 163.068 122.936) (end 164.501001 121.502999) (width 0.25) (layer "B.Cu") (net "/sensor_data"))
 (segment (start 164.501001 121.502999) (end 164.501001 119.951999) (width 0.25) (layer "B.Cu") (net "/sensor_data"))
 (segment (start 166.116 124.46) (end 159.512 124.46) (width 0.25) (layer "F.Cu") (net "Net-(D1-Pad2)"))
 (segment (start 166.5455 122.428) (end 166.5455 124.0305) (width 0.25) (layer "F.Cu") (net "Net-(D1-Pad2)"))
 (segment (start 166.5455 124.0305) (end 166.116 124.46) (width 0.25) (layer "F.Cu") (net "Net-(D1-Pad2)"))
 (segment (start 159.512 124.46) (end 159.055832 124.003832) (width 0.25) (layer "F.Cu") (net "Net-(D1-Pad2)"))
 (segment (start 159.055832 124.003832) (end 159.055832 122.428) (width 0.25) (layer "F.Cu") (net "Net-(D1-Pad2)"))
 (segment (start 142.9281 122.4788) (end 142.9281 124.7694) (width 0.25) (layer "F.Cu") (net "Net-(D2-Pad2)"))
 (segment (start 142.9281 124.7694) (end 144.8031 126.6444) (width 0.25) (layer "F.Cu") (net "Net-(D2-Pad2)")))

